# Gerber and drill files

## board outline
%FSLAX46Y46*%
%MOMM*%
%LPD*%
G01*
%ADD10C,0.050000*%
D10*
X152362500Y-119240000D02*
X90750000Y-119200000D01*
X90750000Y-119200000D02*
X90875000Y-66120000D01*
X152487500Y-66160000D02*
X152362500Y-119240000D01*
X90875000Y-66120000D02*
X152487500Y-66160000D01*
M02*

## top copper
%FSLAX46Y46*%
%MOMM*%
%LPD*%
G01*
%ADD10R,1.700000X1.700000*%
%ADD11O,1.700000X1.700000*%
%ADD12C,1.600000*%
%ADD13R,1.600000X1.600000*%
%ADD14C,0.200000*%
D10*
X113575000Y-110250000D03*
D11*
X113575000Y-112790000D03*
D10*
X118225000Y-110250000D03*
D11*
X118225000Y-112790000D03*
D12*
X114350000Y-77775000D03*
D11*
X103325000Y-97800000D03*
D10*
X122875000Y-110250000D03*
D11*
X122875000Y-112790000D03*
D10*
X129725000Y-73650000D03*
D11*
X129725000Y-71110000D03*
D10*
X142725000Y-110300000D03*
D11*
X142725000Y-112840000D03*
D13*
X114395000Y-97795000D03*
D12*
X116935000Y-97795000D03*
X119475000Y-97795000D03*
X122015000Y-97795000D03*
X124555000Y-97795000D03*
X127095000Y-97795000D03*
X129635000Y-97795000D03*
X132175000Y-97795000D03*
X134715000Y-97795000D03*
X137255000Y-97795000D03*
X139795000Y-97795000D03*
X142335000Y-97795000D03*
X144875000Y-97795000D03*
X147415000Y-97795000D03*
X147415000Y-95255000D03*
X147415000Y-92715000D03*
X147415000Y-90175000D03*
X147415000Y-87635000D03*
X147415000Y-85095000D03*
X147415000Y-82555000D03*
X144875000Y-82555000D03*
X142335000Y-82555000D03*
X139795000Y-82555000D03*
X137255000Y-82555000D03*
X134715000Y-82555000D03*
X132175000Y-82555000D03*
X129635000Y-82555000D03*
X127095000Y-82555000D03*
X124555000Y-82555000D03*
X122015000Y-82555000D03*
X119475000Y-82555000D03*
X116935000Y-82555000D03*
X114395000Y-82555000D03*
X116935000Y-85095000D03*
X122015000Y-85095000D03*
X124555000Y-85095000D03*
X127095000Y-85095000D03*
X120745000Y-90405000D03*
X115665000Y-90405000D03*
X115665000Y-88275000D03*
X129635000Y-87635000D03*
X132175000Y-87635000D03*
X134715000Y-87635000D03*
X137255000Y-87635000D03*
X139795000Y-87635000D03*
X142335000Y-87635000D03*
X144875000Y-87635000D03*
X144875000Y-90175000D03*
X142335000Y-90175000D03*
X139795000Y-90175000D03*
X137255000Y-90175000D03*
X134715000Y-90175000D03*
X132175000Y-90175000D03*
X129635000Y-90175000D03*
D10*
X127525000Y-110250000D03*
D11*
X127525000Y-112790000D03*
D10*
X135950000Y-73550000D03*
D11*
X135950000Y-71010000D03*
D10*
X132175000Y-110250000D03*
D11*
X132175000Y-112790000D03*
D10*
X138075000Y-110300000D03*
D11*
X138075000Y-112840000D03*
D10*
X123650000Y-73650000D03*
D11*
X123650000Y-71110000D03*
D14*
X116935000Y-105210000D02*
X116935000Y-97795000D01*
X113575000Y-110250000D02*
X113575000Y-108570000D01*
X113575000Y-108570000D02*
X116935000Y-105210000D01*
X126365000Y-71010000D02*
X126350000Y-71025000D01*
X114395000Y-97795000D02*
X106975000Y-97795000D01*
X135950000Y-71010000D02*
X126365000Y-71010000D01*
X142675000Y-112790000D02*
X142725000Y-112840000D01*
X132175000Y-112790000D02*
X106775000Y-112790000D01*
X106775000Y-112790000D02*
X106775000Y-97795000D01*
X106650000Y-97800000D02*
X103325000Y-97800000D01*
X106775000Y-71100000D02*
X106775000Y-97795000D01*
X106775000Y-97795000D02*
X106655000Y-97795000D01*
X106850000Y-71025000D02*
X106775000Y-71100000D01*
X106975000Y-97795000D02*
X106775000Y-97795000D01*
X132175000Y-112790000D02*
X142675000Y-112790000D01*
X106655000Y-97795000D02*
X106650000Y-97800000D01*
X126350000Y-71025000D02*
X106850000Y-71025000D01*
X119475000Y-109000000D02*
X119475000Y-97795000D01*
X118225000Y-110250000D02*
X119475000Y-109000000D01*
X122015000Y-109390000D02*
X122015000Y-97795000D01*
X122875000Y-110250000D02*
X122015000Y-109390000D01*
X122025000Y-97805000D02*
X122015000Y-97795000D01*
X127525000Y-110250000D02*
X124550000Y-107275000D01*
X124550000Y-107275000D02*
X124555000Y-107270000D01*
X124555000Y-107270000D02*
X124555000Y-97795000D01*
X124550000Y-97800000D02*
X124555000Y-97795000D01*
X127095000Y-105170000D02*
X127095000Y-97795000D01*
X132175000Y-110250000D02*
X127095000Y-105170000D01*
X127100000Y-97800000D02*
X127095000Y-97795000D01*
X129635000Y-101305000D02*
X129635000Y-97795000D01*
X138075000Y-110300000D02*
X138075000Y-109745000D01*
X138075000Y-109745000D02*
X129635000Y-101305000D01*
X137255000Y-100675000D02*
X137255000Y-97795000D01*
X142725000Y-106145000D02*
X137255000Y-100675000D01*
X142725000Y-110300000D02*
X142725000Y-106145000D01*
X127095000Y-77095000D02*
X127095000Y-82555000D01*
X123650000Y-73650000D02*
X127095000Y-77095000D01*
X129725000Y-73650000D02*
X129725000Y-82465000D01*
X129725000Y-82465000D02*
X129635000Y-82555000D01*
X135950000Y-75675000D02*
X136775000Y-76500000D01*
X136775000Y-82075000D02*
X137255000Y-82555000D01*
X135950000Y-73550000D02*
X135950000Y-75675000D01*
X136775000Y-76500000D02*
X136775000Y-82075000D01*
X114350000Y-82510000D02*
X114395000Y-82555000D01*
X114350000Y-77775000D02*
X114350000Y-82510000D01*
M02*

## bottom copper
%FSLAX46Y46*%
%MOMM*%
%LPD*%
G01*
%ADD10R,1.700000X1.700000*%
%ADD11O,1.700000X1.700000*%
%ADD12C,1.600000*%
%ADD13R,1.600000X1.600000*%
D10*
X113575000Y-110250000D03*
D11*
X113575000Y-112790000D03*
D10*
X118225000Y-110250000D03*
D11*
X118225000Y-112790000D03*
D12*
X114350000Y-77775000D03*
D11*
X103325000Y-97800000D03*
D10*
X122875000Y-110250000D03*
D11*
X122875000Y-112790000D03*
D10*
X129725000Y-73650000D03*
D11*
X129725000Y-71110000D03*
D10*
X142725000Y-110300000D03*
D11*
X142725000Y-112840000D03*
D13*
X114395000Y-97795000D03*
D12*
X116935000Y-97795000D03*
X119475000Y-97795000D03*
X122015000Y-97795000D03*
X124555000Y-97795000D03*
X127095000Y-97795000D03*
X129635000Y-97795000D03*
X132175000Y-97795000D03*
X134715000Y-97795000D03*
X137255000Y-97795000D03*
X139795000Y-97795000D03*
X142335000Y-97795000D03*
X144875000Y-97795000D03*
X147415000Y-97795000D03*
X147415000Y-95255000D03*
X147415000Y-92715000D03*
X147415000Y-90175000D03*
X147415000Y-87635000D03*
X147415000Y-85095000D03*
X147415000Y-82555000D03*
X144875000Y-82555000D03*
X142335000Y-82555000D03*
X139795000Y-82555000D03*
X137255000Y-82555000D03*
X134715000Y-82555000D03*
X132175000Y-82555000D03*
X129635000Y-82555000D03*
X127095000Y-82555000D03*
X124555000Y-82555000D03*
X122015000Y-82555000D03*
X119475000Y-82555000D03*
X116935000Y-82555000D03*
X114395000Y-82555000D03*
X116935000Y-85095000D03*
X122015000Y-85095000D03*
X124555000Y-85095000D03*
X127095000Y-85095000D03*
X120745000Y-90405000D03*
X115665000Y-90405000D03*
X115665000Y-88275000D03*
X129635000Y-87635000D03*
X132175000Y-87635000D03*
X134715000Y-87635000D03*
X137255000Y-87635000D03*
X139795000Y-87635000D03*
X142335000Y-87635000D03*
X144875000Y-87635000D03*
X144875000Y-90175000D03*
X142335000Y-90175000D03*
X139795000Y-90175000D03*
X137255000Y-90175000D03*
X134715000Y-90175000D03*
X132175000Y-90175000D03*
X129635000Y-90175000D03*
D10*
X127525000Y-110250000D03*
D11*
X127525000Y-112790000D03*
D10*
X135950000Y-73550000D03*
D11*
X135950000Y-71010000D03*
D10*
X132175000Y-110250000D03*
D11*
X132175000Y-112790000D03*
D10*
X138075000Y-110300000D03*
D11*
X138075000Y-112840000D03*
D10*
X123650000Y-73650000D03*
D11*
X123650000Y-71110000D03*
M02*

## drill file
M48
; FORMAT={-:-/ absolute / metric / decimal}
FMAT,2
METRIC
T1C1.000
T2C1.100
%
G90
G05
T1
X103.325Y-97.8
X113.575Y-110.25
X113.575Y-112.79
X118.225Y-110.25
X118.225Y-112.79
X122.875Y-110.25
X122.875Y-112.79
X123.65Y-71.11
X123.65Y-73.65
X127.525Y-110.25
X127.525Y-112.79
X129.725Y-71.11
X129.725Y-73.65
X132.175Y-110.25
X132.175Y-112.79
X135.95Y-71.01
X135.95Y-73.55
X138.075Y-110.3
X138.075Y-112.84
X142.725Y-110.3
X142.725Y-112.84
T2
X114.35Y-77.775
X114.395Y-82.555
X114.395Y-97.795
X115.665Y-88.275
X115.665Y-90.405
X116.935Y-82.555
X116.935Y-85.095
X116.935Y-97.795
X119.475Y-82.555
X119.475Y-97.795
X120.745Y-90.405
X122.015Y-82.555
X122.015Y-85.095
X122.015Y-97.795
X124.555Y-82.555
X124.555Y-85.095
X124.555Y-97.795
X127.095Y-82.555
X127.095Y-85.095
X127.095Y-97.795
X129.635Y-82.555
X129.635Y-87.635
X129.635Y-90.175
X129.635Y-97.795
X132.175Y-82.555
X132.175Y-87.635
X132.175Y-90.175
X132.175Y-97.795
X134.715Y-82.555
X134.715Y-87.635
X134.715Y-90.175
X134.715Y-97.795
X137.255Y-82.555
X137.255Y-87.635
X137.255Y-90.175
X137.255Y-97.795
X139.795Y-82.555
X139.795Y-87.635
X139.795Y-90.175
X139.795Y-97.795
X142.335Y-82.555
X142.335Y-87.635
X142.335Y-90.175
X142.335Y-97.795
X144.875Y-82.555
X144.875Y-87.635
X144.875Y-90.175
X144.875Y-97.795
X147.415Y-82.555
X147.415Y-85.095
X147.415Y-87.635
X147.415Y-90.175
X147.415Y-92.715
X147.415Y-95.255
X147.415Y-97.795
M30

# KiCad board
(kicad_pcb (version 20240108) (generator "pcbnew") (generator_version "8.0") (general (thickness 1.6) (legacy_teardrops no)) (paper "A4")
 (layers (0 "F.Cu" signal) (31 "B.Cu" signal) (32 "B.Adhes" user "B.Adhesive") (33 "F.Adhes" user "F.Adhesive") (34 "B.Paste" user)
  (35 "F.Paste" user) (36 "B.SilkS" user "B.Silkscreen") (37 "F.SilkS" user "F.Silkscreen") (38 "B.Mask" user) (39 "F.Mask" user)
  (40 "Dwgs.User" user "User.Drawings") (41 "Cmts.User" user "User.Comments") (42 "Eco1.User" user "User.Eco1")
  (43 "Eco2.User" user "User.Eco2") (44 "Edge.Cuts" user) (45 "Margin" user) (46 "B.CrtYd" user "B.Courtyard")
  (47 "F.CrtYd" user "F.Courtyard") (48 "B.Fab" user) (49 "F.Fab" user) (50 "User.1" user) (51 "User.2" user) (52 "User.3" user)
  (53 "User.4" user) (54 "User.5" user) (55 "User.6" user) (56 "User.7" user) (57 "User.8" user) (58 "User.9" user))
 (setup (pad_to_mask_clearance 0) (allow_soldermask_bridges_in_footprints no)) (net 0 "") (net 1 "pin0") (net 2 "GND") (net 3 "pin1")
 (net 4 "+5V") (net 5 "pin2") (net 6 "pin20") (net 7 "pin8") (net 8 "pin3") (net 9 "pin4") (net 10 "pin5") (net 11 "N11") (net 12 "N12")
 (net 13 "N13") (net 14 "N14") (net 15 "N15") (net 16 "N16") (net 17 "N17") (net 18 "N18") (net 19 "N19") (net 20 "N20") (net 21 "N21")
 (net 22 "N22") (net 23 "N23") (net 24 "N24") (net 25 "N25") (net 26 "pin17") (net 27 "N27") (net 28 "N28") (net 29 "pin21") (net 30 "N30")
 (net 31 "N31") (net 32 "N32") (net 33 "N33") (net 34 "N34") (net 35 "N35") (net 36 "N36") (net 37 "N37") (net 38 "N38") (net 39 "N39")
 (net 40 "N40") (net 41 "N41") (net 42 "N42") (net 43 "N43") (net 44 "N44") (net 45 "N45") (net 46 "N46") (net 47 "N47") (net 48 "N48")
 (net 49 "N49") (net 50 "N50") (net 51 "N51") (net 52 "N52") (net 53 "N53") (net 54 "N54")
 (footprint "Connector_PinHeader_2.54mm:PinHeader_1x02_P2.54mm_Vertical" (layer "F.Cu") (at 113.575 110.25)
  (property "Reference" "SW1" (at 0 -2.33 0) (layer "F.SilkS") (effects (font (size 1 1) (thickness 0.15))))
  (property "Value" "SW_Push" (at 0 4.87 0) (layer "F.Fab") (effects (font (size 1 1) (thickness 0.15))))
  (pad "1" thru_hole rect (at 0 0) (size 1.7 1.7) (drill 1) (layers "*.Cu" "*.Mask") (remove_unused_layers no) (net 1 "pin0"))
  (pad "2" thru_hole oval (at 0 2.54) (size 1.7 1.7) (drill 1) (layers "*.Cu" "*.Mask") (remove_unused_layers no) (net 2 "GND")))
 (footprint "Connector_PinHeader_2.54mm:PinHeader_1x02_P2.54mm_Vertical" (layer "F.Cu") (at 118.225 110.25)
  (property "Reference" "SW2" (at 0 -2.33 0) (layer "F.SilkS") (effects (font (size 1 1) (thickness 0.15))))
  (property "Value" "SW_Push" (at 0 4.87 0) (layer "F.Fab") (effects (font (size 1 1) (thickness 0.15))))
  (pad "1" thru_hole rect (at 0 0) (size 1.7 1.7) (drill 1) (layers "*.Cu" "*.Mask") (remove_unused_layers no) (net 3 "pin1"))
  (pad "2" thru_hole oval (at 0 2.54) (size 1.7 1.7) (drill 1) (layers "*.Cu" "*.Mask") (remove_unused_layers no) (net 2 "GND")))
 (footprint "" (layer "F.Cu") (at 114.35 77.775)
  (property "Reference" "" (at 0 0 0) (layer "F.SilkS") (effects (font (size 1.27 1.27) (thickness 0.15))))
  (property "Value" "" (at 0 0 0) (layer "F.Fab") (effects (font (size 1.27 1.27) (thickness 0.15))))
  (pad "33" thru_hole circle (at 0 0) (size 1.6 1.6) (drill 1.1) (layers "*.Cu" "*.Mask") (remove_unused_layers no) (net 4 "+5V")))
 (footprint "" (layer "F.Cu") (at 103.325 97.8)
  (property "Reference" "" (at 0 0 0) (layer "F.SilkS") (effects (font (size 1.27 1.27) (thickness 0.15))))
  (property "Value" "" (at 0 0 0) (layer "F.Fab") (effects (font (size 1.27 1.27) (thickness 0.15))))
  (pad "2" thru_hole oval (at 0 0) (size 1.7 1.7) (drill 1) (layers "*.Cu" "*.Mask") (remove_unused_layers no) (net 2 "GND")))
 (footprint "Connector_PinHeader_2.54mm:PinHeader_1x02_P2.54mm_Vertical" (layer "F.Cu") (at 122.875 110.25)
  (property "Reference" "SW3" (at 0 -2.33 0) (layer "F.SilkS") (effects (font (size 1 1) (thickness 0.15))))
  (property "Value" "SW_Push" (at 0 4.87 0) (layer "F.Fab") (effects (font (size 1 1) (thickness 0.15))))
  (pad "1" thru_hole rect (at 0 0) (size 1.7 1.7) (drill 1) (layers "*.Cu" "*.Mask") (remove_unused_layers no) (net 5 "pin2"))
  (pad "2" thru_hole oval (at 0 2.54) (size 1.7 1.7) (drill 1) (layers "*.Cu" "*.Mask") (remove_unused_layers no) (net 2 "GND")))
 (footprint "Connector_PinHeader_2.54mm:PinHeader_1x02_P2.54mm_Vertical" (layer "F.Cu") (at 129.725 73.65 180)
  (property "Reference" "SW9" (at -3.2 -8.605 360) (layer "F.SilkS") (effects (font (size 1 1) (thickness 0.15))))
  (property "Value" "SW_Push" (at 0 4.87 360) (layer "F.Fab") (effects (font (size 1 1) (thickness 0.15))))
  (pad "1" thru_hole rect (at 0 0 180) (size 1.7 1.7) (drill 1) (layers "*.Cu" "*.Mask") (remove_unused_layers no) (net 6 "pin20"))
  (pad "2" thru_hole oval (at 0 2.54 180) (size 1.7 1.7) (drill 1) (layers "*.Cu" "*.Mask") (remove_unused_layers no) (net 2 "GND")))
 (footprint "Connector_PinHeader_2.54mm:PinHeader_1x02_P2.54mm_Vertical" (layer "F.Cu") (at 142.725 110.3)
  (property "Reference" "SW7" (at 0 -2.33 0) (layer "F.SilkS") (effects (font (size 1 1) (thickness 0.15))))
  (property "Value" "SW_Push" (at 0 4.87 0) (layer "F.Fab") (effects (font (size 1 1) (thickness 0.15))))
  (pad "1" thru_hole rect (at 0 0) (size 1.7 1.7) (drill 1) (layers "*.Cu" "*.Mask") (remove_unused_layers no) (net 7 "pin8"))
  (pad "2" thru_hole oval (at 0 2.54) (size 1.7 1.7) (drill 1) (layers "*.Cu" "*.Mask") (remove_unused_layers no) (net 2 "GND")))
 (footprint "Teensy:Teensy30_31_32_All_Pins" (layer "F.Cu") (at 130.905 90.175)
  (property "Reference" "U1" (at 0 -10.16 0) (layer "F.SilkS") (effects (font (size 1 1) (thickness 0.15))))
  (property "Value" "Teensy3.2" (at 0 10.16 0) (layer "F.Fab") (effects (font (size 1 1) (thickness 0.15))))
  (pad "1" thru_hole rect (at -16.51 7.62) (size 1.6 1.6) (drill 1.1) (layers "*.Cu" "*.Mask") (remove_unused_layers no) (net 2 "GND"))
  (pad "2" thru_hole circle (at -13.97 7.62) (size 1.6 1.6) (drill 1.1) (layers "*.Cu" "*.Mask") (remove_unused_layers no) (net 1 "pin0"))
  (pad "3" thru_hole circle (at -11.43 7.62) (size 1.6 1.6) (drill 1.1) (layers "*.Cu" "*.Mask") (remove_unused_layers no) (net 3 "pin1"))
  (pad "4" thru_hole circle (at -8.89 7.62) (size 1.6 1.6) (drill 1.1) (layers "*.Cu" "*.Mask") (remove_unused_layers no) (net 5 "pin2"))
  (pad "5" thru_hole circle (at -6.35 7.62) (size 1.6 1.6) (drill 1.1) (layers "*.Cu" "*.Mask") (remove_unused_layers no) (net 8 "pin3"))
  (pad "6" thru_hole circle (at -3.81 7.62) (size 1.6 1.6) (drill 1.1) (layers "*.Cu" "*.Mask") (remove_unused_layers no) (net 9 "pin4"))
  (pad "7" thru_hole circle (at -1.27 7.62) (size 1.6 1.6) (drill 1.1) (layers "*.Cu" "*.Mask") (remove_unused_layers no) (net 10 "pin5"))
  (pad "8" thru_hole circle (at 1.27 7.62) (size 1.6 1.6) (drill 1.1) (layers "*.Cu" "*.Mask") (remove_unused_layers no) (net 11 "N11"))
  (pad "9" thru_hole circle (at 3.81 7.62) (size 1.6 1.6) (drill 1.1) (layers "*.Cu" "*.Mask") (remove_unused_layers no) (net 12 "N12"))
  (pad "10" thru_hole circle (at 6.35 7.62) (size 1.6 1.6) (drill 1.1) (layers "*.Cu" "*.Mask") (remove_unused_layers no) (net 7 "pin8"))
  (pad "11" thru_hole circle (at 8.89 7.62) (size 1.6 1.6) (drill 1.1) (layers "*.Cu" "*.Mask") (remove_unused_layers no) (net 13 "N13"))
  (pad "12" thru_hole circle (at 11.43 7.62) (size 1.6 1.6) (drill 1.1) (layers "*.Cu" "*.Mask") (remove_unused_layers no) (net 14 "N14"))
  (pad "13" thru_hole circle (at 13.97 7.62) (size 1.6 1.6) (drill 1.1) (layers "*.Cu" "*.Mask") (remove_unused_layers no) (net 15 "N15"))
  (pad "14" thru_hole circle (at 16.51 7.62) (size 1.6 1.6) (drill 1.1) (layers "*.Cu" "*.Mask") (remove_unused_layers no) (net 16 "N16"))
  (pad "15" thru_hole circle (at 16.51 5.08) (size 1.6 1.6) (drill 1.1) (layers "*.Cu" "*.Mask") (remove_unused_layers no) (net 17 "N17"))
  (pad "16" thru_hole circle (at 16.51 2.54) (size 1.6 1.6) (drill 1.1) (layers "*.Cu" "*.Mask") (remove_unused_layers no) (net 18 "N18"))
  (pad "17" thru_hole circle (at 16.51 0) (size 1.6 1.6) (drill 1.1) (layers "*.Cu" "*.Mask") (remove_unused_layers no) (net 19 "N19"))
  (pad "18" thru_hole circle (at 16.51 -2.54) (size 1.6 1.6) (drill 1.1) (layers "*.Cu" "*.Mask") (remove_unused_layers no) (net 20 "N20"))
  (pad "19" thru_hole circle (at 16.51 -5.08) (size 1.6 1.6) (drill 1.1) (layers "*.Cu" "*.Mask") (remove_unused_layers no) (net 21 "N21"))
  (pad "20" thru_hole circle (at 16.51 -7.62) (size 1.6 1.6) (drill 1.1) (layers "*.Cu" "*.Mask") (remove_unused_layers no) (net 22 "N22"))
  (pad "21" thru_hole circle (at 13.97 -7.62) (size 1.6 1.6) (drill 1.1) (layers "*.Cu" "*.Mask") (remove_unused_layers no) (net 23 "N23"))
  (pad "22" thru_hole circle (at 11.43 -7.62) (size 1.6 1.6) (drill 1.1) (layers "*.Cu" "*.Mask") (remove_unused_layers no) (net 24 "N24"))
  (pad "23" thru_hole circle (at 8.89 -7.62) (size 1.6 1.6) (drill 1.1) (layers "*.Cu" "*.Mask") (remove_unused_layers no) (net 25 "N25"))
  (pad "24" thru_hole circle (at 6.35 -7.62) (size 1.6 1.6) (drill 1.1) (layers "*.Cu" "*.Mask") (remove_unused_layers no) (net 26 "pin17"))
  (pad "25" thru_hole circle (at 3.81 -7.62) (size 1.6 1.6) (drill 1.1) (layers "*.Cu" "*.Mask") (remove_unused_layers no) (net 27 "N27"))
  (pad "26" thru_hole circle (at 1.27 -7.62) (size 1.6 1.6) (drill 1.1) (layers "*.Cu" "*.Mask") (remove_unused_layers no) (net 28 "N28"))
  (pad "27" thru_hole circle (at -1.27 -7.62) (size 1.6 1.6) (drill 1.1) (layers "*.Cu" "*.Mask") (remove_unused_layers no) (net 6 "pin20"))
  (pad "28" thru_hole circle (at -3.81 -7.62) (size 1.6 1.6) (drill 1.1) (layers "*.Cu" "*.Mask") (remove_unused_layers no) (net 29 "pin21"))
  (pad "29" thru_hole circle (at -6.35 -7.62) (size 1.6 1.6) (drill 1.1) (layers "*.Cu" "*.Mask") (remove_unused_layers no) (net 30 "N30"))
  (pad "30" thru_hole circle (at -8.89 -7.62) (size 1.6 1.6) (drill 1.1) (layers "*.Cu" "*.Mask") (remove_unused_layers no) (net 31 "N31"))
  (pad "31" thru_hole circle (at -11.43 -7.62) (size 1.6 1.6) (drill 1.1) (layers "*.Cu" "*.Mask") (remove_unused_layers no) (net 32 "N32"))
  (pad "32" thru_hole circle (at -13.97 -7.62) (size 1.6 1.6) (drill 1.1) (layers "*.Cu" "*.Mask") (remove_unused_layers no) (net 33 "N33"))
  (pad "33" thru_hole circle (at -16.51 -7.62) (size 1.6 1.6) (drill 1.1) (layers "*.Cu" "*.Mask") (remove_unused_layers no) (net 4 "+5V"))
  (pad "34" thru_hole circle (at -13.97 -5.08) (size 1.6 1.6) (drill 1.1) (layers "*.Cu" "*.Mask") (remove_unused_layers no) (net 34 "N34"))
  (pad "35" thru_hole circle (at -8.89 -5.08) (size 1.6 1.6) (drill 1.1) (layers "*.Cu" "*.Mask") (remove_unused_layers no) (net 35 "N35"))
  (pad "36" thru_hole circle (at -6.35 -5.08) (size 1.6 1.6) (drill 1.1) (layers "*.Cu" "*.Mask") (remove_unused_layers no) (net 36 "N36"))
  (pad "37" thru_hole circle (at -3.81 -5.08) (size 1.6 1.6) (drill 1.1) (layers "*.Cu" "*.Mask") (remove_unused_layers no) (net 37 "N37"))
  (pad "38" thru_hole circle (at -10.16 0.23) (size 1.6 1.6) (drill 1.1) (layers "*.Cu" "*.Mask") (remove_unused_layers no) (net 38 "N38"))
  (pad "39" thru_hole circle (at -15.24 0.23) (size 1.6 1.6) (drill 1.1) (layers "*.Cu" "*.Mask") (remove_unused_layers no) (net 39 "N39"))
  (pad "40" thru_hole circle (at -15.24 -1.9) (size 1.6 1.6) (drill 1.1) (layers "*.Cu" "*.Mask") (remove_unused_layers no) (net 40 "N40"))
  (pad "41" thru_hole circle (at -1.27 -2.54) (size 1.6 1.6) (drill 1.1) (layers "*.Cu" "*.Mask") (remove_unused_layers no) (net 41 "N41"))
  (pad "42" thru_hole circle (at 1.27 -2.54) (size 1.6 1.6) (drill 1.1) (layers "*.Cu" "*.Mask") (remove_unused_layers no) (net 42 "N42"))
  (pad "43" thru_hole circle (at 3.81 -2.54) (size 1.6 1.6) (drill 1.1) (layers "*.Cu" "*.Mask") (remove_unused_layers no) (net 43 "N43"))
  (pad "44" thru_hole circle (at 6.35 -2.54 90) (size 1.6 1.6) (drill 1.1) (layers "*.Cu" "*.Mask") (remove_unused_layers no) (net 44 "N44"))
  (pad "45" thru_hole circle (at 8.89 -2.54) (size 1.6 1.6) (drill 1.1) (layers "*.Cu" "*.Mask") (remove_unused_layers no) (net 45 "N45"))
  (pad "46" thru_hole circle (at 11.43 -2.54) (size 1.6 1.6) (drill 1.1) (layers "*.Cu" "*.Mask") (remove_unused_layers no) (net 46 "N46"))
  (pad "47" thru_hole circle (at 13.97 -2.54) (size 1.6 1.6) (drill 1.1) (layers "*.Cu" "*.Mask") (remove_unused_layers no) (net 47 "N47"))
  (pad "48" thru_hole circle (at 13.97 0) (size 1.6 1.6) (drill 1.1) (layers "*.Cu" "*.Mask") (remove_unused_layers no) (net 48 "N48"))
  (pad "49" thru_hole circle (at 11.43 0) (size 1.6 1.6) (drill 1.1) (layers "*.Cu" "*.Mask") (remove_unused_layers no) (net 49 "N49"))
  (pad "50" thru_hole circle (at 8.89 0) (size 1.6 1.6) (drill 1.1) (layers "*.Cu" "*.Mask") (remove_unused_layers no) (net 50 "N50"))
  (pad "51" thru_hole circle (at 6.35 0) (size 1.6 1.6) (drill 1.1) (layers "*.Cu" "*.Mask") (remove_unused_layers no) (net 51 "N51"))
  (pad "52" thru_hole circle (at 3.81 0) (size 1.6 1.6) (drill 1.1) (layers "*.Cu" "*.Mask") (remove_unused_layers no) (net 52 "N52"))
  (pad "53" thru_hole circle (at 1.27 0) (size 1.6 1.6) (drill 1.1) (layers "*.Cu" "*.Mask") (remove_unused_layers no) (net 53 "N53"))
  (pad "54" thru_hole circle (at -1.27 0) (size 1.6 1.6) (drill 1.1) (layers "*.Cu" "*.Mask") (remove_unused_layers no) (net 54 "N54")))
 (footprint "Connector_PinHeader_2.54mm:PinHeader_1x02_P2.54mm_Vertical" (layer "F.Cu") (at 127.525 110.25)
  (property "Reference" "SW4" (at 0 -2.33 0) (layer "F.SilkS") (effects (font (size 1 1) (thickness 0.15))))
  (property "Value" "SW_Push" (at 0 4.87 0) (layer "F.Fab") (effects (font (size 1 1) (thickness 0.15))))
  (pad "1" thru_hole rect (at 0 0) (size 1.7 1.7) (drill 1) (layers "*.Cu" "*.Mask") (remove_unused_layers no) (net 8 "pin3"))
  (pad "2" thru_hole oval (at 0 2.54) (size 1.7 1.7) (drill 1) (layers "*.Cu" "*.Mask") (remove_unused_layers no) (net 2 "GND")))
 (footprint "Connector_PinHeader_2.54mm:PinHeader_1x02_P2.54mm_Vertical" (layer "F.Cu") (at 135.95 73.55 180)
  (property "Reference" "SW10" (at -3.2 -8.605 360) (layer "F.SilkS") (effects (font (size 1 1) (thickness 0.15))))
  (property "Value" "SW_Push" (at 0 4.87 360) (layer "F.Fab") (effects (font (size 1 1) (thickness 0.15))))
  (pad "1" thru_hole rect (at 0 0 180) (size 1.7 1.7) (drill 1) (layers "*.Cu" "*.Mask") (remove_unused_layers no) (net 26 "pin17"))
  (pad "2" thru_hole oval (at 0 2.54 180) (size 1.7 1.7) (drill 1) (layers "*.Cu" "*.Mask") (remove_unused_layers no) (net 2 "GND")))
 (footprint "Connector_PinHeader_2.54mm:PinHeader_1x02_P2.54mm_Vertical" (layer "F.Cu") (at 132.175 110.25)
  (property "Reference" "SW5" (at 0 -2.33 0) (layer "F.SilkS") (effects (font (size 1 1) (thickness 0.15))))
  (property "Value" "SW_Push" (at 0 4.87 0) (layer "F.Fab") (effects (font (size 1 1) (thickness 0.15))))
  (pad "1" thru_hole rect (at 0 0) (size 1.7 1.7) (drill 1) (layers "*.Cu" "*.Mask") (remove_unused_layers no) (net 9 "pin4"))
  (pad "2" thru_hole oval (at 0 2.54) (size 1.7 1.7) (drill 1) (layers "*.Cu" "*.Mask") (remove_unused_layers no) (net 2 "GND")))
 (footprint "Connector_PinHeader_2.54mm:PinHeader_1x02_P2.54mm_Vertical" (layer "F.Cu") (at 138.075 110.3)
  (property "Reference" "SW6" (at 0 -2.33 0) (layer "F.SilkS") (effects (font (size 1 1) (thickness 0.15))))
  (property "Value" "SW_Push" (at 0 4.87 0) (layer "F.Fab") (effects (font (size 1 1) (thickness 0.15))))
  (pad "1" thru_hole rect (at 0 0) (size 1.7 1.7) (drill 1) (layers "*.Cu" "*.Mask") (remove_unused_layers no) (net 10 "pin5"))
  (pad "2" thru_hole oval (at 0 2.54) (size 1.7 1.7) (drill 1) (layers "*.Cu" "*.Mask") (remove_unused_layers no) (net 2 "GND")))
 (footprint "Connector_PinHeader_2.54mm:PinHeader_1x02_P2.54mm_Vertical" (layer "F.Cu") (at 123.65 73.65 180)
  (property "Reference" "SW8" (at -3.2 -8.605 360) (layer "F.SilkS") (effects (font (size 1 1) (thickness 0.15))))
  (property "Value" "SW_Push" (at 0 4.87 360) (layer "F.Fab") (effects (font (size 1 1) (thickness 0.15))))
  (pad "1" thru_hole rect (at 0 0 180) (size 1.7 1.7) (drill 1) (layers "*.Cu" "*.Mask") (remove_unused_layers no) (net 29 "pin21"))
  (pad "2" thru_hole oval (at 0 2.54 180) (size 1.7 1.7) (drill 1) (layers "*.Cu" "*.Mask") (remove_unused_layers no) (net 2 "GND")))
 (gr_line (start 152.3625 119.24) (end 90.75 119.2) (stroke (width 0.05) (type default)) (layer "Edge.Cuts"))
 (gr_line (start 90.75 119.2) (end 90.875 66.12) (stroke (width 0.05) (type default)) (layer "Edge.Cuts"))
 (gr_line (start 152.4875 66.16) (end 152.3625 119.24) (stroke (width 0.05) (type default)) (layer "Edge.Cuts"))
 (gr_line (start 90.875 66.12) (end 152.4875 66.16) (stroke (width 0.05) (type default)) (layer "Edge.Cuts"))
 (segment (start 116.935 105.21) (end 116.935 97.795) (width 0.2) (layer "F.Cu") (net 1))
 (segment (start 113.575 110.25) (end 113.575 108.57) (width 0.2) (layer "F.Cu") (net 1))
 (segment (start 113.575 108.57) (end 116.935 105.21) (width 0.2) (layer "F.Cu") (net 1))
 (segment (start 126.365 71.01) (end 126.35 71.025) (width 0.2) (layer "F.Cu") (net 2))
 (segment (start 114.395 97.795) (end 106.975 97.795) (width 0.2) (layer "F.Cu") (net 2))
 (segment (start 135.95 71.01) (end 126.365 71.01) (width 0.2) (layer "F.Cu") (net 2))
 (segment (start 142.675 112.79) (end 142.725 112.84) (width 0.2) (layer "F.Cu") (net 2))
 (segment (start 132.175 112.79) (end 106.775 112.79) (width 0.2) (layer "F.Cu") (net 2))
 (segment (start 106.775 112.79) (end 106.775 97.795) (width 0.2) (layer "F.Cu") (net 2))
 (segment (start 106.65 97.8) (end 103.325 97.8) (width 0.2) (layer "F.Cu") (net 2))
 (segment (start 106.775 71.1) (end 106.775 97.795) (width 0.2) (layer "F.Cu") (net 2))
 (segment (start 106.775 97.795) (end 106.655 97.795) (width 0.2) (layer "F.Cu") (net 2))
 (segment (start 106.85 71.025) (end 106.775 71.1) (width 0.2) (layer "F.Cu") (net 2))
 (segment (start 106.975 97.795) (end 106.775 97.795) (width 0.2) (layer "F.Cu") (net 2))
 (segment (start 132.175 112.79) (end 142.675 112.79) (width 0.2) (layer "F.Cu") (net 2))
 (segment (start 106.655 97.795) (end 106.65 97.8) (width 0.2) (layer "F.Cu") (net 2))
 (segment (start 126.35 71.025) (end 106.85 71.025) (width 0.2) (layer "F.Cu") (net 2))
 (segment (start 119.475 109) (end 119.475 97.795) (width 0.2) (layer "F.Cu") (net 3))
 (segment (start 118.225 110.25) (end 119.475 109) (width 0.2) (layer "F.Cu") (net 3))
 (segment (start 122.015 109.39) (end 122.015 97.795) (width 0.2) (layer "F.Cu") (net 5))
 (segment (start 122.875 110.25) (end 122.015 109.39) (width 0.2) (layer "F.Cu") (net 5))
 (segment (start 122.025 97.805) (end 122.015 97.795) (width 0.2) (layer "F.Cu") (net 5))
 (segment (start 127.525 110.25) (end 124.55 107.275) (width 0.2) (layer "F.Cu") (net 8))
 (segment (start 124.55 107.275) (end 124.555 107.27) (width 0.2) (layer "F.Cu") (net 8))
 (segment (start 124.555 107.27) (end 124.555 97.795) (width 0.2) (layer "F.Cu") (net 8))
 (segment (start 124.55 97.8) (end 124.555 97.795) (width 0.2) (layer "F.Cu") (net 8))
 (segment (start 127.095 105.17) (end 127.095 97.795) (width 0.2) (layer "F.Cu") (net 9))
 (segment (start 132.175 110.25) (end 127.095 105.17) (width 0.2) (layer "F.Cu") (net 9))
 (segment (start 127.1 97.8) (end 127.095 97.795) (width 0.2) (layer "F.Cu") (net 9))
 (segment (start 129.635 101.305) (end 129.635 97.795) (width 0.2) (layer "F.Cu") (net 10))
 (segment (start 138.075 110.3) (end 138.075 109.745) (width 0.2) (layer "F.Cu") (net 10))
 (segment (start 138.075 109.745) (end 129.635 101.305) (width 0.2) (layer "F.Cu") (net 10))
 (segment (start 137.255 100.675) (end 137.255 97.795) (width 0.2) (layer "F.Cu") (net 7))
 (segment (start 142.725 106.145) (end 137.255 100.675) (width 0.2) (layer "F.Cu") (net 7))
 (segment (start 142.725 110.3) (end 142.725 106.145) (width 0.2) (layer "F.Cu") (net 7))
 (segment (start 127.095 77.095) (end 127.095 82.555) (width 0.2) (layer "F.Cu") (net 29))
 (segment (start 123.65 73.65) (end 127.095 77.095) (width 0.2) (layer "F.Cu") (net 29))
 (segment (start 129.725 73.65) (end 129.725 82.465) (width 0.2) (layer "F.Cu") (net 6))
 (segment (start 129.725 82.465) (end 129.635 82.555) (width 0.2) (layer "F.Cu") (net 6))
 (segment (start 135.95 75.675) (end 136.775 76.5) (width 0.2) (layer "F.Cu") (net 26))
 (segment (start 136.775 82.075) (end 137.255 82.555) (width 0.2) (layer "F.Cu") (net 26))
 (segment (start 135.95 73.55) (end 135.95 75.675) (width 0.2) (layer "F.Cu") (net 26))
 (segment (start 136.775 76.5) (end 136.775 82.075) (width 0.2) (layer "F.Cu") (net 26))
 (segment (start 114.35 82.51) (end 114.395 82.555) (width 0.2) (layer "F.Cu") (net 4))
 (segment (start 114.35 77.775) (end 114.35 82.51) (width 0.2) (layer "F.Cu") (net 4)))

